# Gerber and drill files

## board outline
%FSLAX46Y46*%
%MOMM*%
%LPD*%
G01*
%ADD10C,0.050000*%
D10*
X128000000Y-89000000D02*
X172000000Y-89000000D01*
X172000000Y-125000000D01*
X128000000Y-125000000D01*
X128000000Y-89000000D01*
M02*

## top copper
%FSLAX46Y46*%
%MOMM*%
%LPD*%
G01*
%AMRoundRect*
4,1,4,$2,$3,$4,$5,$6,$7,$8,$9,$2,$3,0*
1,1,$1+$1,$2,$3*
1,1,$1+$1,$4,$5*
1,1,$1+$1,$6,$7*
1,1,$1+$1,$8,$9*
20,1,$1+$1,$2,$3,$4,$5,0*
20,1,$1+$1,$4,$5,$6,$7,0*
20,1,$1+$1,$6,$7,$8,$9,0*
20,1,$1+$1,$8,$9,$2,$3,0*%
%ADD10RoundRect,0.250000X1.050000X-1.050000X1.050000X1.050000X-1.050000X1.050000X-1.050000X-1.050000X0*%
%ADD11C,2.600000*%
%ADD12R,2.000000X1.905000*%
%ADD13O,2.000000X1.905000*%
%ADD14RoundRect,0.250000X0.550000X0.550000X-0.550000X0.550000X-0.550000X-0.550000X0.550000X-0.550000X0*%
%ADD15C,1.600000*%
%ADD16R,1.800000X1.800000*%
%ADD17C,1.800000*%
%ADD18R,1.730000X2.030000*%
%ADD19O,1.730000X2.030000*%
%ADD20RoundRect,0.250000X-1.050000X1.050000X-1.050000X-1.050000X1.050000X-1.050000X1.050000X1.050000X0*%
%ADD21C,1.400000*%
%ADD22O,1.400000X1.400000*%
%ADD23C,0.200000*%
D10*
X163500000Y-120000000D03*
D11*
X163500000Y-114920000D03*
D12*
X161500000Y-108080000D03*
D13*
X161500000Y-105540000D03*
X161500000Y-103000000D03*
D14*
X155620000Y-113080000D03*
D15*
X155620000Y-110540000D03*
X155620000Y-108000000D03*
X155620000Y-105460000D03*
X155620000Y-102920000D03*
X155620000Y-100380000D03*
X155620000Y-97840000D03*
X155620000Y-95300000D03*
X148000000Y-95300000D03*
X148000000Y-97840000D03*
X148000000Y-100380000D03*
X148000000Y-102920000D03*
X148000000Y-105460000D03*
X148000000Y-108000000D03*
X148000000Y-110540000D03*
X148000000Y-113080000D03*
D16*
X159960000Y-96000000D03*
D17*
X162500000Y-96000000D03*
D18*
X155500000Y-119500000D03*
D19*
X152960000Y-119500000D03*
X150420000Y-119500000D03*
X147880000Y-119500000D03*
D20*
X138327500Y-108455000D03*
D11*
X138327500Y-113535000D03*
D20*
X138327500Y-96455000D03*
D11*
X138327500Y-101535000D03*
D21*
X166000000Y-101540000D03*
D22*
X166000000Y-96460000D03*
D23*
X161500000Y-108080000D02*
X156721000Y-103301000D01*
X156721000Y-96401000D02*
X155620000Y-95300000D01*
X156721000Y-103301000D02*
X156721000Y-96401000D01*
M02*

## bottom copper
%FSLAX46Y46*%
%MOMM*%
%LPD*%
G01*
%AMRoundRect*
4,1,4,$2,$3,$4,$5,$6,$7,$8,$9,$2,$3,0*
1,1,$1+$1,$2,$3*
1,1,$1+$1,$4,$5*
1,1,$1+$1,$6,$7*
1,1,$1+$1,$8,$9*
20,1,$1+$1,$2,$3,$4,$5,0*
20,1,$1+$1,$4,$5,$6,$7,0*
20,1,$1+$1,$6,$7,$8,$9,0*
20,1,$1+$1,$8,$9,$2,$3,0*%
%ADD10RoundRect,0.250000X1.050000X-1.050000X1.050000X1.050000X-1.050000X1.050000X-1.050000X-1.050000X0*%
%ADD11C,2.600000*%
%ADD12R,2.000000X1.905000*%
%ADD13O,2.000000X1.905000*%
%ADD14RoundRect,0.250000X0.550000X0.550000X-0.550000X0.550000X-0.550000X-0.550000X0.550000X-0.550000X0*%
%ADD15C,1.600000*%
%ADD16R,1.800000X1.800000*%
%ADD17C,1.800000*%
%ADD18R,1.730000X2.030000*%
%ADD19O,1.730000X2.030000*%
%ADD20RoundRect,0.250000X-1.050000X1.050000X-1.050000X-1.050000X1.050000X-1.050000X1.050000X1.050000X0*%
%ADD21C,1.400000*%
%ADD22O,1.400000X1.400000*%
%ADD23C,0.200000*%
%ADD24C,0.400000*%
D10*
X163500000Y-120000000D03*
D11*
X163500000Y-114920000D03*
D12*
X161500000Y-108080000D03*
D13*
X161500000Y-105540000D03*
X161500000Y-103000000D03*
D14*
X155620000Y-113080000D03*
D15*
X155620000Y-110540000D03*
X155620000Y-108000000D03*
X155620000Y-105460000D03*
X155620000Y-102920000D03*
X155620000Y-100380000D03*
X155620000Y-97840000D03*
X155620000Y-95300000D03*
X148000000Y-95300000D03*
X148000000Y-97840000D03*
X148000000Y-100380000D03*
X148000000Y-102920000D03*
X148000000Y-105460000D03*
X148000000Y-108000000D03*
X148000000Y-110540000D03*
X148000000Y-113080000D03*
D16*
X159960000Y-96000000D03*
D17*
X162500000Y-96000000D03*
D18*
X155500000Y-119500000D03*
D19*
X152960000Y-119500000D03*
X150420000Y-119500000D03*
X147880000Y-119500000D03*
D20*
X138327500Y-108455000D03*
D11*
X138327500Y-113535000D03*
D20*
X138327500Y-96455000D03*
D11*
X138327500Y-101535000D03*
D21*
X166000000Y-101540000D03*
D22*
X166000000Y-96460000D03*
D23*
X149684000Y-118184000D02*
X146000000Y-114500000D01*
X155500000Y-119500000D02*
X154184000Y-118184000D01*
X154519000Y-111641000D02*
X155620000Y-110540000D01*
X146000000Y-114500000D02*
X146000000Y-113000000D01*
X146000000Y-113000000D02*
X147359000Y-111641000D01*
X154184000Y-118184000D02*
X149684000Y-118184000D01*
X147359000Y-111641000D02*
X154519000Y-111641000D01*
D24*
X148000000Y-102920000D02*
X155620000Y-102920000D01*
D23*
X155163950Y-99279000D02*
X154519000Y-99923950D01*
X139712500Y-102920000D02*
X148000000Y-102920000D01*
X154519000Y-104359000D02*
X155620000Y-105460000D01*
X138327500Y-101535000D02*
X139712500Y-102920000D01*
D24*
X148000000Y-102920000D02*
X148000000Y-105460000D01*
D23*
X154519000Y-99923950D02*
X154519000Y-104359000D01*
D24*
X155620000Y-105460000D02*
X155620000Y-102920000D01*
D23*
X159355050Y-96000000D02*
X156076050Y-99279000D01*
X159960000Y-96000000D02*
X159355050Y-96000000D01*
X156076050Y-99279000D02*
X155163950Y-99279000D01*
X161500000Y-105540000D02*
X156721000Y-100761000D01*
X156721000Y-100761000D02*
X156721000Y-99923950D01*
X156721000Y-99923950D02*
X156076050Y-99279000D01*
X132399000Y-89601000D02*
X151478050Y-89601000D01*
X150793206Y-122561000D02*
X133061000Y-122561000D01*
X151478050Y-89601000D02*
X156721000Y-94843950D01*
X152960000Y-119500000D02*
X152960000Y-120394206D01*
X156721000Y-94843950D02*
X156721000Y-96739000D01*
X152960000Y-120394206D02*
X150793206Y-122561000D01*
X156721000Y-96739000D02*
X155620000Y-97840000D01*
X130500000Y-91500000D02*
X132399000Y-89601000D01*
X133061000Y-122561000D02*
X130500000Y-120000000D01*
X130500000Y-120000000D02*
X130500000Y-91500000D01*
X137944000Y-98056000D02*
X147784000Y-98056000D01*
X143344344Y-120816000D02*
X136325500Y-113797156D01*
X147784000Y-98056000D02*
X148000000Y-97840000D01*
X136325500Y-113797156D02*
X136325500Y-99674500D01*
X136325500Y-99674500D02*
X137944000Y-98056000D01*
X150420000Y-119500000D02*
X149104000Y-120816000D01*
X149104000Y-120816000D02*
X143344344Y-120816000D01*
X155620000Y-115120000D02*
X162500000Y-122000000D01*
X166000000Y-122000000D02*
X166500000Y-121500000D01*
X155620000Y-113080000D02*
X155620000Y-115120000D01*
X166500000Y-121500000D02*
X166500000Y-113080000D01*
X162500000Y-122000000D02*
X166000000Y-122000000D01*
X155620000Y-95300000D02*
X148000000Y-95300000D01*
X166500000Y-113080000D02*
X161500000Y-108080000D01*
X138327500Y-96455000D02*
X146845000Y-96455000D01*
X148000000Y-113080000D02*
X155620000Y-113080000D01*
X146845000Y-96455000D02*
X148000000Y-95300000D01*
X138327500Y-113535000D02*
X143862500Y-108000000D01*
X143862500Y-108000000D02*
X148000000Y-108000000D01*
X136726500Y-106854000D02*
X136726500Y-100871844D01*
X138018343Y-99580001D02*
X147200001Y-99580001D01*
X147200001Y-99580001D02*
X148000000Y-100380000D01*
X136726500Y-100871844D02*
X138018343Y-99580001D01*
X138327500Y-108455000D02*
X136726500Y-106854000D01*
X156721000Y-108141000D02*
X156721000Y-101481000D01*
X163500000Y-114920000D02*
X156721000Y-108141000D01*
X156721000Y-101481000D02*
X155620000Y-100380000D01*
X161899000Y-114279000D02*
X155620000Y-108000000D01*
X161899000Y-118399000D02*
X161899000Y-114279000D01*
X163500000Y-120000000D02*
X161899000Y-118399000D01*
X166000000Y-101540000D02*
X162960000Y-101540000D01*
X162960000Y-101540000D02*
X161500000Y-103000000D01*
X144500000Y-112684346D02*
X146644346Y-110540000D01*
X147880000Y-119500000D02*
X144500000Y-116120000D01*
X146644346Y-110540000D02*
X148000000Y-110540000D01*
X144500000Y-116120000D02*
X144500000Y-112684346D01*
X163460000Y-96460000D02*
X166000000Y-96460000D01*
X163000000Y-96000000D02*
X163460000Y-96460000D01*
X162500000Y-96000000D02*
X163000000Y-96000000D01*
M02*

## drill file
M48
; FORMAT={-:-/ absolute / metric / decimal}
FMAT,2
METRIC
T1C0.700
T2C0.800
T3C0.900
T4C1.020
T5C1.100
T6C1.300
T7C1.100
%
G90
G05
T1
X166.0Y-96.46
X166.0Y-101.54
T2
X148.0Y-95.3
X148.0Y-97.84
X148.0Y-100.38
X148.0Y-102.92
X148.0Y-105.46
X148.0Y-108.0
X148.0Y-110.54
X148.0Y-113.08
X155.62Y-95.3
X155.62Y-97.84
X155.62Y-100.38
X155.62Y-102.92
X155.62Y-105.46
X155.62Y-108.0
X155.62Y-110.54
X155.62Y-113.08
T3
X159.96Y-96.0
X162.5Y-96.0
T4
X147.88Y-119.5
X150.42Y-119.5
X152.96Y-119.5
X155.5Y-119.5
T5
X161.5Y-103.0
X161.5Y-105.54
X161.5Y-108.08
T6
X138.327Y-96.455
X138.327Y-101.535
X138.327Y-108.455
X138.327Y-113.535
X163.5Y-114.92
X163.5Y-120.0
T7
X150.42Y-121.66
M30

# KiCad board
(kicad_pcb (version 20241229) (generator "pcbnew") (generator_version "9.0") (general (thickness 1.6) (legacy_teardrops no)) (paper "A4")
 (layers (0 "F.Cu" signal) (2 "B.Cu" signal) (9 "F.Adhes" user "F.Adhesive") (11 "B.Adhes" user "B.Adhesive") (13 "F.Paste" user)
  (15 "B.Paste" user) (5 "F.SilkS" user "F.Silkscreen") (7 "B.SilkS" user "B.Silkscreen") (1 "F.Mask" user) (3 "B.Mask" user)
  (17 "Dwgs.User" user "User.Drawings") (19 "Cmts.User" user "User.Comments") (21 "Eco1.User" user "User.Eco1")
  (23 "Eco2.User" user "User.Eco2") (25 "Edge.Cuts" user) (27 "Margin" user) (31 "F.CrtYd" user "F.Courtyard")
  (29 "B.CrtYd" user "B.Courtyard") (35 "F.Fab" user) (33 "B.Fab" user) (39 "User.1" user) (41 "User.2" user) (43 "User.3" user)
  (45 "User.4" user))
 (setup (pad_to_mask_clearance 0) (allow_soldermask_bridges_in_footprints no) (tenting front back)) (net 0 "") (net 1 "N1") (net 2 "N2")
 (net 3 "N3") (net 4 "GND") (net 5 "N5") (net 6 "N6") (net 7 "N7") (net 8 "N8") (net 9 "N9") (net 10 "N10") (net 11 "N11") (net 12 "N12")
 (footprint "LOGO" (layer "F.Cu") (at 169 93)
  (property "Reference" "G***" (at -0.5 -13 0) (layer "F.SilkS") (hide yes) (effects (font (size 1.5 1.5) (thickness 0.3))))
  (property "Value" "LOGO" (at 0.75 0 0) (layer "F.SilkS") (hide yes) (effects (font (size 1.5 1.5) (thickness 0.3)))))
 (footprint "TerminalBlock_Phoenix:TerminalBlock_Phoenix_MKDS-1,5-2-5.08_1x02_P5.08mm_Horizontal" (layer "F.Cu") (at 163.5 120 90)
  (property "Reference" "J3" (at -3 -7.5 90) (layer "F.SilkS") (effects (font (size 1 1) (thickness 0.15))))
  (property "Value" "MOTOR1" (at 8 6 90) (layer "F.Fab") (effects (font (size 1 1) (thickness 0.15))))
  (pad "1" thru_hole roundrect (at 0 0 90) (size 2.6 2.6) (drill 1.3) (layers "*.Cu" "*.Mask") (remove_unused_layers no)
   (roundrect_rratio 0.096154) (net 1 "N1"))
  (pad "2" thru_hole circle (at 5.08 0 90) (size 2.6 2.6) (drill 1.3) (layers "*.Cu" "*.Mask") (remove_unused_layers no) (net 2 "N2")))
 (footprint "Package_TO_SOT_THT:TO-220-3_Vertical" (layer "F.Cu") (at 161.5 108.08 90)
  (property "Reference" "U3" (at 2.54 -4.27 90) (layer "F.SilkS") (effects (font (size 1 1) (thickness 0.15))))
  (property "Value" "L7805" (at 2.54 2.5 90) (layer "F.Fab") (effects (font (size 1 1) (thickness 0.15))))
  (pad "1" thru_hole rect (at 0 0 90) (size 1.905 2) (drill 1.1) (layers "*.Cu" "*.Mask") (remove_unused_layers no) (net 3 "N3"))
  (pad "2" thru_hole oval (at 2.54 0 90) (size 1.905 2) (drill 1.1) (layers "*.Cu" "*.Mask") (remove_unused_layers no) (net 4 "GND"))
  (pad "3" thru_hole oval (at 5.08 0 90) (size 1.905 2) (drill 1.1) (layers "*.Cu" "*.Mask") (remove_unused_layers no) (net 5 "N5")))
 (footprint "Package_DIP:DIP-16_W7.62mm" (layer "F.Cu") (at 155.62 113.08 180)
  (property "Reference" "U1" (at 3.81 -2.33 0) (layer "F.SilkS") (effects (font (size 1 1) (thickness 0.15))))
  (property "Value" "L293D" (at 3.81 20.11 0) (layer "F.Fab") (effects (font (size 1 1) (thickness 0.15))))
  (pad "1" thru_hole roundrect (at 0 0 180) (size 1.6 1.6) (drill 0.8) (layers "*.Cu" "*.Mask") (remove_unused_layers no)
   (roundrect_rratio 0.15625) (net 3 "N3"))
  (pad "2" thru_hole circle (at 0 2.54 180) (size 1.6 1.6) (drill 0.8) (layers "*.Cu" "*.Mask") (remove_unused_layers no) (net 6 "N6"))
  (pad "3" thru_hole circle (at 0 5.08 180) (size 1.6 1.6) (drill 0.8) (layers "*.Cu" "*.Mask") (remove_unused_layers no) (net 1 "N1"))
  (pad "4" thru_hole circle (at 0 7.62 180) (size 1.6 1.6) (drill 0.8) (layers "*.Cu" "*.Mask") (remove_unused_layers no) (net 4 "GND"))
  (pad "5" thru_hole circle (at 0 10.16 180) (size 1.6 1.6) (drill 0.8) (layers "*.Cu" "*.Mask") (remove_unused_layers no) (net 4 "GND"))
  (pad "6" thru_hole circle (at 0 12.7 180) (size 1.6 1.6) (drill 0.8) (layers "*.Cu" "*.Mask") (remove_unused_layers no) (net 2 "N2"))
  (pad "7" thru_hole circle (at 0 15.24 180) (size 1.6 1.6) (drill 0.8) (layers "*.Cu" "*.Mask") (remove_unused_layers no) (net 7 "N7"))
  (pad "8" thru_hole circle (at 0 17.78 180) (size 1.6 1.6) (drill 0.8) (layers "*.Cu" "*.Mask") (remove_unused_layers no) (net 3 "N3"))
  (pad "9" thru_hole circle (at 7.62 17.78 180) (size 1.6 1.6) (drill 0.8) (layers "*.Cu" "*.Mask") (remove_unused_layers no) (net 3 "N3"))
  (pad "10" thru_hole circle (at 7.62 15.24 180) (size 1.6 1.6) (drill 0.8) (layers "*.Cu" "*.Mask") (remove_unused_layers no) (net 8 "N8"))
  (pad "11" thru_hole circle (at 7.62 12.7 180) (size 1.6 1.6) (drill 0.8) (layers "*.Cu" "*.Mask") (remove_unused_layers no) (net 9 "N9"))
  (pad "12" thru_hole circle (at 7.62 10.16 180) (size 1.6 1.6) (drill 0.8) (layers "*.Cu" "*.Mask") (remove_unused_layers no) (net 4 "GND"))
  (pad "13" thru_hole circle (at 7.62 7.62 180) (size 1.6 1.6) (drill 0.8) (layers "*.Cu" "*.Mask") (remove_unused_layers no) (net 4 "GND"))
  (pad "14" thru_hole circle (at 7.62 5.08 180) (size 1.6 1.6) (drill 0.8) (layers "*.Cu" "*.Mask") (remove_unused_layers no) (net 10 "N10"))
  (pad "15" thru_hole circle (at 7.62 2.54 180) (size 1.6 1.6) (drill 0.8) (layers "*.Cu" "*.Mask") (remove_unused_layers no) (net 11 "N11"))
  (pad "16" thru_hole circle (at 7.62 0 180) (size 1.6 1.6) (drill 0.8) (layers "*.Cu" "*.Mask") (remove_unused_layers no) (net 3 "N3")))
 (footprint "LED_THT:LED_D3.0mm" (layer "F.Cu") (at 159.96 96)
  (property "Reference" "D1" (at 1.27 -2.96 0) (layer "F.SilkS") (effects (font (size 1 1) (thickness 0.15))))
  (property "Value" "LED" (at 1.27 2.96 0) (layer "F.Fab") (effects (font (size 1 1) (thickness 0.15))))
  (pad "1" thru_hole rect (at 0 0) (size 1.8 1.8) (drill 0.9) (layers "*.Cu" "*.Mask") (remove_unused_layers no) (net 4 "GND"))
  (pad "2" thru_hole circle (at 2.54 0) (size 1.8 1.8) (drill 0.9) (layers "*.Cu" "*.Mask") (remove_unused_layers no) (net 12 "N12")))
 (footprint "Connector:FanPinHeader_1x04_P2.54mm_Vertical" (layer "F.Cu") (at 155.5 119.5 180)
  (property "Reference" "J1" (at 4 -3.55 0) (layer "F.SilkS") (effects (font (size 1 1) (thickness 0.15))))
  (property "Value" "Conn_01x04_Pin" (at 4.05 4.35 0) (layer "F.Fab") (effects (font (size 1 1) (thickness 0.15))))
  (pad "" np_thru_hole circle (at 5.08 -2.16 270) (size 1.1 1.1) (drill 1.1) (layers "*.Cu" "*.Mask"))
  (pad "1" thru_hole rect (at 0 0 270) (size 2.03 1.73) (drill 1.02) (layers "*.Cu" "*.Mask") (remove_unused_layers no) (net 6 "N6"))
  (pad "2" thru_hole oval (at 2.54 0 270) (size 2.03 1.73) (drill 1.02) (layers "*.Cu" "*.Mask") (remove_unused_layers no) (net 7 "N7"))
  (pad "3" thru_hole oval (at 5.08 0 270) (size 2.03 1.73) (drill 1.02) (layers "*.Cu" "*.Mask") (remove_unused_layers no) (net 8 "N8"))
  (pad "4" thru_hole oval (at 7.62 0 270) (size 2.03 1.73) (drill 1.02) (layers "*.Cu" "*.Mask") (remove_unused_layers no) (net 11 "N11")))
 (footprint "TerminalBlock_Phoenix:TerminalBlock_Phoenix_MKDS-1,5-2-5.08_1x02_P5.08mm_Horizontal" (layer "F.Cu") (at 138.3275 108.455 -90)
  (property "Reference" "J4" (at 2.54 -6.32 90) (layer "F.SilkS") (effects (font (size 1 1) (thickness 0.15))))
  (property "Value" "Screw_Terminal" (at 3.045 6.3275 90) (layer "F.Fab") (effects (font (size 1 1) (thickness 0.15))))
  (pad "1" thru_hole roundrect (at 0 0 270) (size 2.6 2.6) (drill 1.3) (layers "*.Cu" "*.Mask") (remove_unused_layers no)
   (roundrect_rratio 0.096154) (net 9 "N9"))
  (pad "2" thru_hole circle (at 5.08 0 270) (size 2.6 2.6) (drill 1.3) (layers "*.Cu" "*.Mask") (remove_unused_layers no) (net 10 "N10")))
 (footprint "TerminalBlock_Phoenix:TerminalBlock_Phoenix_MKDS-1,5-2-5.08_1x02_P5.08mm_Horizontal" (layer "F.Cu") (at 138.3275 96.455 -90)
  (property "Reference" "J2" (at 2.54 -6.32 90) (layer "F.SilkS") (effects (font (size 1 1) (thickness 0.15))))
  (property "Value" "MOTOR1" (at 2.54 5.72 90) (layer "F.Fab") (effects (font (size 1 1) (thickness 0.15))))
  (pad "1" thru_hole roundrect (at 0 0 270) (size 2.6 2.6) (drill 1.3) (layers "*.Cu" "*.Mask") (remove_unused_layers no)
   (roundrect_rratio 0.096154) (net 3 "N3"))
  (pad "2" thru_hole circle (at 5.08 0 270) (size 2.6 2.6) (drill 1.3) (layers "*.Cu" "*.Mask") (remove_unused_layers no) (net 4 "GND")))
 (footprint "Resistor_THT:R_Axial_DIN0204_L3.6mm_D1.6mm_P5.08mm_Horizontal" (layer "F.Cu") (at 166 101.54 90)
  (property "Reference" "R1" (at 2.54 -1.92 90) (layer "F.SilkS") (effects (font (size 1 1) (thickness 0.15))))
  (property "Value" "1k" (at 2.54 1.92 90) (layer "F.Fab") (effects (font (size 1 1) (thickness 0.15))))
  (pad "1" thru_hole circle (at 0 0 90) (size 1.4 1.4) (drill 0.7) (layers "*.Cu" "*.Mask") (remove_unused_layers no) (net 5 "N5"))
  (pad "2" thru_hole oval (at 5.08 0 90) (size 1.4 1.4) (drill 0.7) (layers "*.Cu" "*.Mask") (remove_unused_layers no) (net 12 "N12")))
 (gr_rect (start 128 89) (end 172 125) (stroke (width 0.05) (type default)) (fill no) (layer "Edge.Cuts"))
 (segment (start 149.684 118.184) (end 146 114.5) (width 0.2) (layer "B.Cu") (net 6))
 (segment (start 155.5 119.5) (end 154.184 118.184) (width 0.2) (layer "B.Cu") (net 6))
 (segment (start 154.519 111.641) (end 155.62 110.54) (width 0.2) (layer "B.Cu") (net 6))
 (segment (start 146 114.5) (end 146 113) (width 0.2) (layer "B.Cu") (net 6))
 (segment (start 146 113) (end 147.359 111.641) (width 0.2) (layer "B.Cu") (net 6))
 (segment (start 154.184 118.184) (end 149.684 118.184) (width 0.2) (layer "B.Cu") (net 6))
 (segment (start 147.359 111.641) (end 154.519 111.641) (width 0.2) (layer "B.Cu") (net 6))
 (segment (start 148 102.92) (end 155.62 102.92) (width 0.4) (layer "B.Cu") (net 4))
 (segment (start 155.16395 99.279) (end 154.519 99.92395) (width 0.2) (layer "B.Cu") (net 4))
 (segment (start 139.7125 102.92) (end 148 102.92) (width 0.2) (layer "B.Cu") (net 4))
 (segment (start 154.519 104.359) (end 155.62 105.46) (width 0.2) (layer "B.Cu") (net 4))
 (segment (start 138.3275 101.535) (end 139.7125 102.92) (width 0.2) (layer "B.Cu") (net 4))
 (segment (start 148 102.92) (end 148 105.46) (width 0.4) (layer "B.Cu") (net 4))
 (segment (start 154.519 99.92395) (end 154.519 104.359) (width 0.2) (layer "B.Cu") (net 4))
 (segment (start 155.62 105.46) (end 155.62 102.92) (width 0.4) (layer "B.Cu") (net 4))
 (segment (start 159.35505 96) (end 156.07605 99.279) (width 0.2) (layer "B.Cu") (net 4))
 (segment (start 159.96 96) (end 159.35505 96) (width 0.2) (layer "B.Cu") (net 4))
 (segment (start 156.07605 99.279) (end 155.16395 99.279) (width 0.2) (layer "B.Cu") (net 4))
 (segment (start 161.5 105.54) (end 156.721 100.761) (width 0.2) (layer "B.Cu") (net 4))
 (segment (start 156.721 100.761) (end 156.721 99.92395) (width 0.2) (layer "B.Cu") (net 4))
 (segment (start 156.721 99.92395) (end 156.07605 99.279) (width 0.2) (layer "B.Cu") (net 4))
 (segment (start 132.399 89.601) (end 151.47805 89.601) (width 0.2) (layer "B.Cu") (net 7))
 (segment (start 150.793206 122.561) (end 133.061 122.561) (width 0.2) (layer "B.Cu") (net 7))
 (segment (start 151.47805 89.601) (end 156.721 94.84395) (width 0.2) (layer "B.Cu") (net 7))
 (segment (start 152.96 119.5) (end 152.96 120.394206) (width 0.2) (layer "B.Cu") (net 7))
 (segment (start 156.721 94.84395) (end 156.721 96.739) (width 0.2) (layer "B.Cu") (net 7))
 (segment (start 152.96 120.394206) (end 150.793206 122.561) (width 0.2) (layer "B.Cu") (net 7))
 (segment (start 156.721 96.739) (end 155.62 97.84) (width 0.2) (layer "B.Cu") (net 7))
 (segment (start 130.5 91.5) (end 132.399 89.601) (width 0.2) (layer "B.Cu") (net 7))
 (segment (start 133.061 122.561) (end 130.5 120) (width 0.2) (layer "B.Cu") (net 7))
 (segment (start 130.5 120) (end 130.5 91.5) (width 0.2) (layer "B.Cu") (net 7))
 (segment (start 137.944 98.056) (end 147.784 98.056) (width 0.2) (layer "B.Cu") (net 8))
 (segment (start 143.344344 120.816) (end 136.3255 113.797156) (width 0.2) (layer "B.Cu") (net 8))
 (segment (start 147.784 98.056) (end 148 97.84) (width 0.2) (layer "B.Cu") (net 8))
 (segment (start 136.3255 113.797156) (end 136.3255 99.6745) (width 0.2) (layer "B.Cu") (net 8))
 (segment (start 136.3255 99.6745) (end 137.944 98.056) (width 0.2) (layer "B.Cu") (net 8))
 (segment (start 150.42 119.5) (end 149.104 120.816) (width 0.2) (layer "B.Cu") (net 8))
 (segment (start 149.104 120.816) (end 143.344344 120.816) (width 0.2) (layer "B.Cu") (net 8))
 (segment (start 161.5 108.08) (end 156.721 103.301) (width 0.2) (layer "F.Cu") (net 3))
 (segment (start 156.721 96.401) (end 155.62 95.3) (width 0.2) (layer "F.Cu") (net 3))
 (segment (start 156.721 103.301) (end 156.721 96.401) (width 0.2) (layer "F.Cu") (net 3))
 (segment (start 155.62 115.12) (end 162.5 122) (width 0.2) (layer "B.Cu") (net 3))
 (segment (start 166 122) (end 166.5 121.5) (width 0.2) (layer "B.Cu") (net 3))
 (segment (start 155.62 113.08) (end 155.62 115.12) (width 0.2) (layer "B.Cu") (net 3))
 (segment (start 166.5 121.5) (end 166.5 113.08) (width 0.2) (layer "B.Cu") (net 3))
 (segment (start 162.5 122) (end 166 122) (width 0.2) (layer "B.Cu") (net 3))
 (segment (start 155.62 95.3) (end 148 95.3) (width 0.2) (layer "B.Cu") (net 3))
 (segment (start 166.5 113.08) (end 161.5 108.08) (width 0.2) (layer "B.Cu") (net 3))
 (segment (start 138.3275 96.455) (end 146.845 96.455) (width 0.2) (layer "B.Cu") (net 3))
 (segment (start 148 113.08) (end 155.62 113.08) (width 0.2) (layer "B.Cu") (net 3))
 (segment (start 146.845 96.455) (end 148 95.3) (width 0.2) (layer "B.Cu") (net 3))
 (segment (start 138.3275 113.535) (end 143.8625 108) (width 0.2) (layer "B.Cu") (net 10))
 (segment (start 143.8625 108) (end 148 108) (width 0.2) (layer "B.Cu") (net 10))
 (segment (start 136.7265 106.854) (end 136.7265 100.871844) (width 0.2) (layer "B.Cu") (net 9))
 (segment (start 138.018343 99.580001) (end 147.200001 99.580001) (width 0.2) (layer "B.Cu") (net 9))
 (segment (start 147.200001 99.580001) (end 148 100.38) (width 0.2) (layer "B.Cu") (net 9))
 (segment (start 136.7265 100.871844) (end 138.018343 99.580001) (width 0.2) (layer "B.Cu") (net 9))
 (segment (start 138.3275 108.455) (end 136.7265 106.854) (width 0.2) (layer "B.Cu") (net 9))
 (segment (start 156.721 108.141) (end 156.721 101.481) (width 0.2) (layer "B.Cu") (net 2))
 (segment (start 163.5 114.92) (end 156.721 108.141) (width 0.2) (layer "B.Cu") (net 2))
 (segment (start 156.721 101.481) (end 155.62 100.38) (width 0.2) (layer "B.Cu") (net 2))
 (segment (start 161.899 114.279) (end 155.62 108) (width 0.2) (layer "B.Cu") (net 1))
 (segment (start 161.899 118.399) (end 161.899 114.279) (width 0.2) (layer "B.Cu") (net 1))
 (segment (start 163.5 120) (end 161.899 118.399) (width 0.2) (layer "B.Cu") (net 1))
 (segment (start 166 101.54) (end 162.96 101.54) (width 0.2) (layer "B.Cu") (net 5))
 (segment (start 162.96 101.54) (end 161.5 103) (width 0.2) (layer "B.Cu") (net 5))
 (segment (start 144.5 112.684346) (end 146.644346 110.54) (width 0.2) (layer "B.Cu") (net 11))
 (segment (start 147.88 119.5) (end 144.5 116.12) (width 0.2) (layer "B.Cu") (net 11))
 (segment (start 146.644346 110.54) (end 148 110.54) (width 0.2) (layer "B.Cu") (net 11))
 (segment (start 144.5 116.12) (end 144.5 112.684346) (width 0.2) (layer "B.Cu") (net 11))
 (segment (start 163.46 96.46) (end 166 96.46) (width 0.2) (layer "B.Cu") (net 12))
 (segment (start 163 96) (end 163.46 96.46) (width 0.2) (layer "B.Cu") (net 12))
 (segment (start 162.5 96) (end 163 96) (width 0.2) (layer "B.Cu") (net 12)))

